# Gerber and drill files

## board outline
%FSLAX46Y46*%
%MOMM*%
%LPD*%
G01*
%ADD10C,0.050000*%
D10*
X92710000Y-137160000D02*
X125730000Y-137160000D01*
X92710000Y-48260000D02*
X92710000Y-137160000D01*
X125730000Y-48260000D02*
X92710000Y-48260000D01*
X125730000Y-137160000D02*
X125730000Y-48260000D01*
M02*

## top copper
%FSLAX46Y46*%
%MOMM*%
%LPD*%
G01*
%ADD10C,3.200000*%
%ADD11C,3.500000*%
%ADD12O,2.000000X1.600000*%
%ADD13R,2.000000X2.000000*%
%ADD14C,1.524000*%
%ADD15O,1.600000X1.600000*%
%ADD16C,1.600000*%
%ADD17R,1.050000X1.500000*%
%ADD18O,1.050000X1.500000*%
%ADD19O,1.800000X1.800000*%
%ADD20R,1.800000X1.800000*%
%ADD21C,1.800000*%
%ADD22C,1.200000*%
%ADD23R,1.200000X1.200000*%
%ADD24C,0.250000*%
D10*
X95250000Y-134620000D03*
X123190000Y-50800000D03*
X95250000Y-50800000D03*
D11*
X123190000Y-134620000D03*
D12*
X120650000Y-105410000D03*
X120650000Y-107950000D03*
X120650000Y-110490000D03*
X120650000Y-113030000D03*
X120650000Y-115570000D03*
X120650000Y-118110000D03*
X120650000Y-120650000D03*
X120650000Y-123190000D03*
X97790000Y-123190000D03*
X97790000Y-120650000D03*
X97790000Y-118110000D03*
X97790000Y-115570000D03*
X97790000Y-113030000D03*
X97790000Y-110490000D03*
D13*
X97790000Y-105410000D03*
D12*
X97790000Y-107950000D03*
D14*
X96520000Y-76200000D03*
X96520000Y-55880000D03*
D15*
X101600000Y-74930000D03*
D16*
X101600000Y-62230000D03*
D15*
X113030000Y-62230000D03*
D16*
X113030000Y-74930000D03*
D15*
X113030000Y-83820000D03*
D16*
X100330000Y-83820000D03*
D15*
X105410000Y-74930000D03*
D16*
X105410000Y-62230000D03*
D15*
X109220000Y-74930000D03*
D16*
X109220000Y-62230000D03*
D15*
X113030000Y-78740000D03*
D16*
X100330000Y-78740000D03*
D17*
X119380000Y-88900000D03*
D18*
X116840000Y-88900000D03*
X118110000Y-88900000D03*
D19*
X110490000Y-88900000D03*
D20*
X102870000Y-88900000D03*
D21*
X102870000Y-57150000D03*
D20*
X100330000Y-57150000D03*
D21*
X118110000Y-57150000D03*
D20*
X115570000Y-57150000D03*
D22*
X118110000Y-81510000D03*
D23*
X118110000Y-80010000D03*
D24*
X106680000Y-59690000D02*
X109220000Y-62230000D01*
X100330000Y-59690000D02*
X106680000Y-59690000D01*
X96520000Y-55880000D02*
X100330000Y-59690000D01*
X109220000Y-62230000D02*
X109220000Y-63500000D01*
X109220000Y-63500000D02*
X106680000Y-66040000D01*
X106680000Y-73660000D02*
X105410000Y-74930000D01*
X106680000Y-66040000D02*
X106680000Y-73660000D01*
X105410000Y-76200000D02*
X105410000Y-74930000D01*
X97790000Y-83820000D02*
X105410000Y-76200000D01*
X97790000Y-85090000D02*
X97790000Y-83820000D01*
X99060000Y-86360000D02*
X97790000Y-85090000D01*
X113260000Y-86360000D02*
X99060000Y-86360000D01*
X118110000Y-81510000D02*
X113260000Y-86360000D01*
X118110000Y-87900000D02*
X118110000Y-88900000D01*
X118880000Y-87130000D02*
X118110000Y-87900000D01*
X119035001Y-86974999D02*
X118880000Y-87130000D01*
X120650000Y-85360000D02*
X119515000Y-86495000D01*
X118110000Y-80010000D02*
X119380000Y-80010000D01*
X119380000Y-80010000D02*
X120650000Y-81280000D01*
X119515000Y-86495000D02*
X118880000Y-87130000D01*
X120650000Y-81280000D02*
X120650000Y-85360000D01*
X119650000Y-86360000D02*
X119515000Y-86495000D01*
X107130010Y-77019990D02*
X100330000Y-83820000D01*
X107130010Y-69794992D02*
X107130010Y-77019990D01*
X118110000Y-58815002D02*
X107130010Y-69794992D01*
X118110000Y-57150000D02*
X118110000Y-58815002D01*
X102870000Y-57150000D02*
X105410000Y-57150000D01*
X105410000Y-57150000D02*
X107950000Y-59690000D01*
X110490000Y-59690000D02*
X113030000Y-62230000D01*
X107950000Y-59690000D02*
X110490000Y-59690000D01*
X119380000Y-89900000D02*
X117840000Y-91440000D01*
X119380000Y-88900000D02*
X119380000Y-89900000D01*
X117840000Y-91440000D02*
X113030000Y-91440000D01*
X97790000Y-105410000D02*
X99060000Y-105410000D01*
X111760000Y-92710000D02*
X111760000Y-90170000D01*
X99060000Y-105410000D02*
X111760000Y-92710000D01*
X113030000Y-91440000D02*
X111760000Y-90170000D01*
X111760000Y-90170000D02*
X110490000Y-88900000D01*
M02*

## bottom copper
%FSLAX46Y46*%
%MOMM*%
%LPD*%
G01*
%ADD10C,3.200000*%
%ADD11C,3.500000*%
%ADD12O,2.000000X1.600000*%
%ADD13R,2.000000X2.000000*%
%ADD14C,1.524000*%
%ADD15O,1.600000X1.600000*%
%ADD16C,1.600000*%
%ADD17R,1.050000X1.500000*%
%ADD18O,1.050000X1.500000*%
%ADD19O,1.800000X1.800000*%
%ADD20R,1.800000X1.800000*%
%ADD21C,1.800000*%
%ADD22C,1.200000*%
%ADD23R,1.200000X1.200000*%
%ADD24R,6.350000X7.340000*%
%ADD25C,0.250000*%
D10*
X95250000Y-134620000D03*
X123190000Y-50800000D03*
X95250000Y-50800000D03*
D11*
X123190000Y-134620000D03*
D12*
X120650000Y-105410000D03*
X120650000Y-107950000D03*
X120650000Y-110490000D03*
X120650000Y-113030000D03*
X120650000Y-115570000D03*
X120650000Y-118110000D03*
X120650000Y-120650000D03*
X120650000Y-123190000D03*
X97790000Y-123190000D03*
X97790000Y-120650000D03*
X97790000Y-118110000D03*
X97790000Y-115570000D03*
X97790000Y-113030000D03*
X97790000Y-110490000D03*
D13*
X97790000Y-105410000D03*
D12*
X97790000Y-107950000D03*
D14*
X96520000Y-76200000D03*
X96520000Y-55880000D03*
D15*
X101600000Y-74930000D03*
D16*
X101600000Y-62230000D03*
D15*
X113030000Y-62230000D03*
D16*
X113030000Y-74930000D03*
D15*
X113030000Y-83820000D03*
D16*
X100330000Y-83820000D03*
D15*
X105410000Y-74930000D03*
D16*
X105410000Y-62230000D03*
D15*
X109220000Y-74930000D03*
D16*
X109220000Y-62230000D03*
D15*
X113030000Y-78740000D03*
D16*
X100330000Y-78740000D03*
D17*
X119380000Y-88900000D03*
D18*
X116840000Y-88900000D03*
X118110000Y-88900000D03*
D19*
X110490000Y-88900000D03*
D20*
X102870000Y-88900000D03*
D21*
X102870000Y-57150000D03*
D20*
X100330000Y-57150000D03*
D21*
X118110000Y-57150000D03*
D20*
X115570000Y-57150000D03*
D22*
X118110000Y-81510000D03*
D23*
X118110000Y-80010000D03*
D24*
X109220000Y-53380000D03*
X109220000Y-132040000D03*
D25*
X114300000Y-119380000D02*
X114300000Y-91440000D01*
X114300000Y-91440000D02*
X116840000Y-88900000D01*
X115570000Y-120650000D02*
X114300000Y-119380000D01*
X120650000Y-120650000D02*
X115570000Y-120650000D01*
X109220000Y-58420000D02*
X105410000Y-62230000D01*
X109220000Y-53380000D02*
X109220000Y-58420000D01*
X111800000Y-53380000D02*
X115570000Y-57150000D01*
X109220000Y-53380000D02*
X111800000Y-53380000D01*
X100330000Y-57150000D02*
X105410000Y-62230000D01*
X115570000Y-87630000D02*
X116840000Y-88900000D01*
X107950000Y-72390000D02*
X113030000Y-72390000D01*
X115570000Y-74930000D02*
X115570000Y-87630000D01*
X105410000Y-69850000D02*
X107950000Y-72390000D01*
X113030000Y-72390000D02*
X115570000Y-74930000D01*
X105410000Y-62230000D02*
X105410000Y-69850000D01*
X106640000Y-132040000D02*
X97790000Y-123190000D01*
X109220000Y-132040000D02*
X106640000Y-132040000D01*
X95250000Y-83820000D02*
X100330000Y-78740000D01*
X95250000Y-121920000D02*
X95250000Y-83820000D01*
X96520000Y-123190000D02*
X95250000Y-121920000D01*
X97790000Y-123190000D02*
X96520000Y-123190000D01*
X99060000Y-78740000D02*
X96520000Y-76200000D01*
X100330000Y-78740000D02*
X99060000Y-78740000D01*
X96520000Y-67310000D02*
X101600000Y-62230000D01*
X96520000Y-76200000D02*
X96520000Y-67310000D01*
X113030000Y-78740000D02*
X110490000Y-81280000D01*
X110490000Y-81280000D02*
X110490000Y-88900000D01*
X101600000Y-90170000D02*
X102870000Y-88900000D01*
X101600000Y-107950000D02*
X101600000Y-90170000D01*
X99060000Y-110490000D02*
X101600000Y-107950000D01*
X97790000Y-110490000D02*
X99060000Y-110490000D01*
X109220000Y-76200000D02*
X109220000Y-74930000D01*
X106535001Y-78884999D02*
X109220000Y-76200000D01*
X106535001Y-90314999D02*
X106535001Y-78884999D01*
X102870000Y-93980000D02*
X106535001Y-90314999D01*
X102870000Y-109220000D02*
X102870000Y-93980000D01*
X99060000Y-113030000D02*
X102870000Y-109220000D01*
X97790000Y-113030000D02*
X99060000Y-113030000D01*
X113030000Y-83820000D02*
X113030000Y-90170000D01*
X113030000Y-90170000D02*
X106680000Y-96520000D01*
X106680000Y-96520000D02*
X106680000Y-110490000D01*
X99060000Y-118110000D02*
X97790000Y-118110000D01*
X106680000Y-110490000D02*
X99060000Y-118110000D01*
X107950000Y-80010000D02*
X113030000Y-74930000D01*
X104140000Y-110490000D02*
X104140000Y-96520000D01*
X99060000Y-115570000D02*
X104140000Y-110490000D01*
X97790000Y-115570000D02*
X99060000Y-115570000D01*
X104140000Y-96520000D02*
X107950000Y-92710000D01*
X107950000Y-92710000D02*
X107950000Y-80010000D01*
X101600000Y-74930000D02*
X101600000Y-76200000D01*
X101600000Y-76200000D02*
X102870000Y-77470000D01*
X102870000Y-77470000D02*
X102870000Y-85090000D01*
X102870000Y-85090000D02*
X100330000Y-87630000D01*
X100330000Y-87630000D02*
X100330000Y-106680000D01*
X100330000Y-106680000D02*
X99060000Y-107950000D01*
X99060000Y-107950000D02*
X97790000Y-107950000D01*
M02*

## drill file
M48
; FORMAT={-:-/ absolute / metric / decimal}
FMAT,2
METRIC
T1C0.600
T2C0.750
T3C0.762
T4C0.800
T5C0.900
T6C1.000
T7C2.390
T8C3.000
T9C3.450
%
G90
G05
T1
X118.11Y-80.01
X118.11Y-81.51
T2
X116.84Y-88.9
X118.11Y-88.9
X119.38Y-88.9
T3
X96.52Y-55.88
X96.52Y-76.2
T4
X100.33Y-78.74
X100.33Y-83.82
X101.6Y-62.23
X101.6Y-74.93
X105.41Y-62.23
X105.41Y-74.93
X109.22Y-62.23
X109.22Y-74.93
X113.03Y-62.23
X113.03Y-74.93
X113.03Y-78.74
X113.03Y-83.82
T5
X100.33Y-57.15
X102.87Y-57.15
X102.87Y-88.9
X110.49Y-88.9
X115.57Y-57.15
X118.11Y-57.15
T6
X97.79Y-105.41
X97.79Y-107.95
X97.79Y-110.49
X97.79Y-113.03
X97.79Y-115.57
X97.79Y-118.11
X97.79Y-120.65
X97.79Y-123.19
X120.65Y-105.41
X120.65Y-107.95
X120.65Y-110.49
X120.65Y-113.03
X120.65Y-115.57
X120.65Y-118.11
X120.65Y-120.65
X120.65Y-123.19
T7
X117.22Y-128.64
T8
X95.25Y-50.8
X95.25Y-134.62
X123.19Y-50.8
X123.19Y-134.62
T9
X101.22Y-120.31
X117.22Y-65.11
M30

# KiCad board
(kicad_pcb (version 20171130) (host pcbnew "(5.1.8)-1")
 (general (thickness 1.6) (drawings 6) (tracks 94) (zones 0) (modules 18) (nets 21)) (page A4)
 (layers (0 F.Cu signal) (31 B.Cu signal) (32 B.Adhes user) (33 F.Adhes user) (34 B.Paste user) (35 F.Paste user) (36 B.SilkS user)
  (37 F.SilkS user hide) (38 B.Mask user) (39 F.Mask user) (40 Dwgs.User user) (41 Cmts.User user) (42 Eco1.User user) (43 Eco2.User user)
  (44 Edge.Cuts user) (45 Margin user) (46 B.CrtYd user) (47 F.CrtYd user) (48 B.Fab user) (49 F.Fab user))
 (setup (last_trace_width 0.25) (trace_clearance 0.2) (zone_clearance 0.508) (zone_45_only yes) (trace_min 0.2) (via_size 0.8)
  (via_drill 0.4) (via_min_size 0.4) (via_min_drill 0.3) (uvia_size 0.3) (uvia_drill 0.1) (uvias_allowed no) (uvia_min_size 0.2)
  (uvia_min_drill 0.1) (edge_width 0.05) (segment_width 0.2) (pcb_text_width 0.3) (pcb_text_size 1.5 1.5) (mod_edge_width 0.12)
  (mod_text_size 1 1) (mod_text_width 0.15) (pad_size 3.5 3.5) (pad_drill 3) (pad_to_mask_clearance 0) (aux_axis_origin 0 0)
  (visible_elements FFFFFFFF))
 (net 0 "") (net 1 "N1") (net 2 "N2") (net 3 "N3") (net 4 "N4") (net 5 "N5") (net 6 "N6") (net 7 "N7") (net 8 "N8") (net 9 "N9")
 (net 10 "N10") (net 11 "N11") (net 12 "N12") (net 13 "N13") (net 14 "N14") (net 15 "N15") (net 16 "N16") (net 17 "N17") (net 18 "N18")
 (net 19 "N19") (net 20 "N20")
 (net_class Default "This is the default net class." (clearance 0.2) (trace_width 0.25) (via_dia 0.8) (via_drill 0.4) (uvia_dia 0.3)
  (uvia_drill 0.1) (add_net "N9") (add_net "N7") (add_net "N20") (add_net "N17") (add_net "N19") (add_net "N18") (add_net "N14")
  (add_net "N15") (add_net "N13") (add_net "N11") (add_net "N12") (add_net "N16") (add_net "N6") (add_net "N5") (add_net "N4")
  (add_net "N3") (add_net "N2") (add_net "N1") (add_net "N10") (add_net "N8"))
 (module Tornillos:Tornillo (layer F.Cu) (at 95.25 132.08)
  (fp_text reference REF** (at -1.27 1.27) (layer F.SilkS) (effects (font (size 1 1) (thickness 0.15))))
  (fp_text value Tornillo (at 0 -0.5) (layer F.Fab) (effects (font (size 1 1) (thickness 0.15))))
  (pad "" np_thru_hole circle (at 0 2.54) (size 3.2 3.2) (drill 3) (layers *.Cu *.Mask)))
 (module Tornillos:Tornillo (layer F.Cu) (at 123.19 48.26)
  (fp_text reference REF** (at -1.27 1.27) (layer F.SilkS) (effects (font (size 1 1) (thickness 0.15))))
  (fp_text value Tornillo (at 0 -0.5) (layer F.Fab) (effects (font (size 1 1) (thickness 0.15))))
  (pad "" np_thru_hole circle (at 0 2.54) (size 3.2 3.2) (drill 3) (layers *.Cu *.Mask)))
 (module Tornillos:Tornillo (layer F.Cu) (at 95.25 48.26)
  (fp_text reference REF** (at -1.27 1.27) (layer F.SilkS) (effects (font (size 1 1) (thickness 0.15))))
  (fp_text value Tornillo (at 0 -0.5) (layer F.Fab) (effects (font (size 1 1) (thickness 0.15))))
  (pad "" np_thru_hole circle (at 0 2.54) (size 3.2 3.2) (drill 3) (layers *.Cu *.Mask)))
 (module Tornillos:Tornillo (layer F.Cu) (at 123.19 132.08)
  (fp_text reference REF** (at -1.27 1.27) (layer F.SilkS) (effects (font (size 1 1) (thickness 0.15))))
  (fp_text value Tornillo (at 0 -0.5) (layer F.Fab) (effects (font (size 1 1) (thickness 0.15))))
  (pad "" np_thru_hole circle (at 0 2.54) (size 3.5 3.5) (drill 3) (layers *.Cu *.Mask)))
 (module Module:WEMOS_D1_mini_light (layer F.Cu) (at 97.79 105.41)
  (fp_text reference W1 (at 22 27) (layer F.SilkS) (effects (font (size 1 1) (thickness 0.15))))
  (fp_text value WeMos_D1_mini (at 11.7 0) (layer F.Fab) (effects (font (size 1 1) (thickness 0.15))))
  (pad 16 thru_hole oval (at 22.86 0) (size 2 1.6) (drill 1) (layers *.Cu *.Mask) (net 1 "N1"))
  (pad 15 thru_hole oval (at 22.86 2.54) (size 2 1.6) (drill 1) (layers *.Cu *.Mask) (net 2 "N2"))
  (pad 14 thru_hole oval (at 22.86 5.08) (size 2 1.6) (drill 1) (layers *.Cu *.Mask) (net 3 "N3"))
  (pad 13 thru_hole oval (at 22.86 7.62) (size 2 1.6) (drill 1) (layers *.Cu *.Mask) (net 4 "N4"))
  (pad 12 thru_hole oval (at 22.86 10.16) (size 2 1.6) (drill 1) (layers *.Cu *.Mask) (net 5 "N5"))
  (pad 11 thru_hole oval (at 22.86 12.7) (size 2 1.6) (drill 1) (layers *.Cu *.Mask) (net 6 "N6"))
  (pad 10 thru_hole oval (at 22.86 15.24) (size 2 1.6) (drill 1) (layers *.Cu *.Mask) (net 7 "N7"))
  (pad 9 thru_hole oval (at 22.86 17.78) (size 2 1.6) (drill 1) (layers *.Cu *.Mask) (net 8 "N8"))
  (pad 8 thru_hole oval (at 0 17.78) (size 2 1.6) (drill 1) (layers *.Cu *.Mask) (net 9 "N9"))
  (pad 7 thru_hole oval (at 0 15.24) (size 2 1.6) (drill 1) (layers *.Cu *.Mask) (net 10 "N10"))
  (pad 6 thru_hole oval (at 0 12.7) (size 2 1.6) (drill 1) (layers *.Cu *.Mask) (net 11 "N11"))
  (pad 5 thru_hole oval (at 0 10.16) (size 2 1.6) (drill 1) (layers *.Cu *.Mask) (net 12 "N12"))
  (pad 4 thru_hole oval (at 0 7.62) (size 2 1.6) (drill 1) (layers *.Cu *.Mask) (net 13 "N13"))
  (pad 3 thru_hole oval (at 0 5.08) (size 2 1.6) (drill 1) (layers *.Cu *.Mask) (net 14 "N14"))
  (pad 1 thru_hole rect (at 0 0) (size 2 2) (drill 1) (layers *.Cu *.Mask) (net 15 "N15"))
  (pad 2 thru_hole oval (at 0 2.54) (size 2 1.6) (drill 1) (layers *.Cu *.Mask) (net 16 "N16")))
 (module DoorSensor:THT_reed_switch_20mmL (layer F.Cu) (at 100.33 63.5 270)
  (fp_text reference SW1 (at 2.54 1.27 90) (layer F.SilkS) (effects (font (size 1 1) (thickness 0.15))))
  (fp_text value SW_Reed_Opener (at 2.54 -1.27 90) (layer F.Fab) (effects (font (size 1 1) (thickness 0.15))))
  (pad 2 thru_hole circle (at 12.7 3.81 270) (size 1.524 1.524) (drill 0.762) (layers *.Cu *.Mask) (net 9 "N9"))
  (pad 1 thru_hole circle (at -7.62 3.81 270) (size 1.524 1.524) (drill 0.762) (layers *.Cu *.Mask) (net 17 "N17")))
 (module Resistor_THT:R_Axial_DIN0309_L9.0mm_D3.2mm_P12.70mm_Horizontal (layer F.Cu) (at 101.6 62.23 270)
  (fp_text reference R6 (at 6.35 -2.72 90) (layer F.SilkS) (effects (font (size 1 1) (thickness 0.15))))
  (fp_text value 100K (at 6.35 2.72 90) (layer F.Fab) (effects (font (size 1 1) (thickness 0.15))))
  (pad 2 thru_hole oval (at 12.7 0 270) (size 1.6 1.6) (drill 0.8) (layers *.Cu *.Mask) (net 16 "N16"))
  (pad 1 thru_hole circle (at 0 0 270) (size 1.6 1.6) (drill 0.8) (layers *.Cu *.Mask) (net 9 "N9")))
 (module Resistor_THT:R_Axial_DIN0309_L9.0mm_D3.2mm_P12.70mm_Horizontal (layer F.Cu) (at 113.03 74.93 90)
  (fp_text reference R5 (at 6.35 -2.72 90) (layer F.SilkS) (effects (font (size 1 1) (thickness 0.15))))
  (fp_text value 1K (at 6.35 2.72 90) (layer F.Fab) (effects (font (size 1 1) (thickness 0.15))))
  (pad 2 thru_hole oval (at 12.7 0 90) (size 1.6 1.6) (drill 0.8) (layers *.Cu *.Mask) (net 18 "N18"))
  (pad 1 thru_hole circle (at 0 0 90) (size 1.6 1.6) (drill 0.8) (layers *.Cu *.Mask) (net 12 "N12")))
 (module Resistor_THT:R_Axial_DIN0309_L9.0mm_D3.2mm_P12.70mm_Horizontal (layer F.Cu) (at 100.33 83.82)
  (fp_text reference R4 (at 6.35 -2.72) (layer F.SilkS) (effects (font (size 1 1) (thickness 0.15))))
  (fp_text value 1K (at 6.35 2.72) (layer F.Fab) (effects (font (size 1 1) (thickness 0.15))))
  (pad 2 thru_hole oval (at 12.7 0) (size 1.6 1.6) (drill 0.8) (layers *.Cu *.Mask) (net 11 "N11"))
  (pad 1 thru_hole circle (at 0 0) (size 1.6 1.6) (drill 0.8) (layers *.Cu *.Mask) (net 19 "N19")))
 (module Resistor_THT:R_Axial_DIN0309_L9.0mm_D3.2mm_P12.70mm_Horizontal (layer F.Cu) (at 105.41 62.23 270)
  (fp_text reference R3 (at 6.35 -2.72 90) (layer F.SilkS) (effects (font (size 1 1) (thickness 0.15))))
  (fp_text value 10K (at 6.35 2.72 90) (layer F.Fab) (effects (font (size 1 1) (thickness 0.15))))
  (pad 2 thru_hole oval (at 12.7 0 270) (size 1.6 1.6) (drill 0.8) (layers *.Cu *.Mask) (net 17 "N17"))
  (pad 1 thru_hole circle (at 0 0 270) (size 1.6 1.6) (drill 0.8) (layers *.Cu *.Mask) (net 7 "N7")))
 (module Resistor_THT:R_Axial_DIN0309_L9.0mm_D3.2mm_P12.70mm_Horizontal (layer F.Cu) (at 109.22 62.23 270)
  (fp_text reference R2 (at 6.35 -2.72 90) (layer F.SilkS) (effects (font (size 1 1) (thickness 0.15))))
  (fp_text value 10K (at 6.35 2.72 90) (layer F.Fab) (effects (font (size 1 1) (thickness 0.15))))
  (pad 2 thru_hole oval (at 12.7 0 270) (size 1.6 1.6) (drill 0.8) (layers *.Cu *.Mask) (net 13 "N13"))
  (pad 1 thru_hole circle (at 0 0 270) (size 1.6 1.6) (drill 0.8) (layers *.Cu *.Mask) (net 17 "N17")))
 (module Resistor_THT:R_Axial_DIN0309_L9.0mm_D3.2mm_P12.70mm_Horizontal (layer F.Cu) (at 100.33 78.74)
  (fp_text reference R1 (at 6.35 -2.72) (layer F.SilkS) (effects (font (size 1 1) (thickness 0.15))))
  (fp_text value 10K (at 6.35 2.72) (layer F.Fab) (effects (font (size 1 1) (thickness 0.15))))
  (pad 2 thru_hole oval (at 12.7 0) (size 1.6 1.6) (drill 0.8) (layers *.Cu *.Mask) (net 15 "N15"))
  (pad 1 thru_hole circle (at 0 0) (size 1.6 1.6) (drill 0.8) (layers *.Cu *.Mask) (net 9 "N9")))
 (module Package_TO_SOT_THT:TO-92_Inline (layer F.Cu) (at 119.38 88.9 180)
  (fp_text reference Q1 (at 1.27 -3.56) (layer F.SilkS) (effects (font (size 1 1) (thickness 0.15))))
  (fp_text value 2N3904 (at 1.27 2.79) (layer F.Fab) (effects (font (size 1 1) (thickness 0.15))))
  (pad 1 thru_hole rect (at 0 0 180) (size 1.05 1.5) (drill 0.75) (layers *.Cu *.Mask) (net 15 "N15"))
  (pad 3 thru_hole oval (at 2.54 0 180) (size 1.05 1.5) (drill 0.75) (layers *.Cu *.Mask) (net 7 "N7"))
  (pad 2 thru_hole oval (at 1.27 0 180) (size 1.05 1.5) (drill 0.75) (layers *.Cu *.Mask) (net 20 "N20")))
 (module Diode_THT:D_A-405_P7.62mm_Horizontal (layer F.Cu) (at 102.87 88.9)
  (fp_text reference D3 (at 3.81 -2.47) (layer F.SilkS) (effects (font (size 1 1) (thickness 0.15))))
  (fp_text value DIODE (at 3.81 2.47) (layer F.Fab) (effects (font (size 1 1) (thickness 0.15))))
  (pad 2 thru_hole oval (at 7.62 0) (size 1.8 1.8) (drill 0.9) (layers *.Cu *.Mask) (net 15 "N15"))
  (pad 1 thru_hole rect (at 0 0) (size 1.8 1.8) (drill 0.9) (layers *.Cu *.Mask) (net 14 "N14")))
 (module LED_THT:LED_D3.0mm (layer F.Cu) (at 100.33 57.15)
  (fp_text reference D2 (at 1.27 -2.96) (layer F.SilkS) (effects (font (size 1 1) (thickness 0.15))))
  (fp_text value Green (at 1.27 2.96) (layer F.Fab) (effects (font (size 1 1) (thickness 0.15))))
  (pad 2 thru_hole circle (at 2.54 0) (size 1.8 1.8) (drill 0.9) (layers *.Cu *.Mask) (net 18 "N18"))
  (pad 1 thru_hole rect (at 0 0) (size 1.8 1.8) (drill 0.9) (layers *.Cu *.Mask) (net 7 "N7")))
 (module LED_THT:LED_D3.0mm (layer F.Cu) (at 115.57 57.15)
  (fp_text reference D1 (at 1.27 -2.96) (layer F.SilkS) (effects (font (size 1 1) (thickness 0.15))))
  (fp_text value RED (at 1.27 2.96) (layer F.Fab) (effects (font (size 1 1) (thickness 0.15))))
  (pad 2 thru_hole circle (at 2.54 0) (size 1.8 1.8) (drill 0.9) (layers *.Cu *.Mask) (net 19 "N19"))
  (pad 1 thru_hole rect (at 0 0) (size 1.8 1.8) (drill 0.9) (layers *.Cu *.Mask) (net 7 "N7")))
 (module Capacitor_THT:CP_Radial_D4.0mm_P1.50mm (layer F.Cu) (at 118.11 80.01 270)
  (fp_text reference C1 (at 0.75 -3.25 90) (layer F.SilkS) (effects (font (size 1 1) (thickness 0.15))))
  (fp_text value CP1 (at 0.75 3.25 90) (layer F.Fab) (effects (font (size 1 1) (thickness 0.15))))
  (pad 2 thru_hole circle (at 1.5 0 270) (size 1.2 1.2) (drill 0.6) (layers *.Cu *.Mask) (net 17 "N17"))
  (pad 1 thru_hole rect (at 0 0 270) (size 1.2 1.2) (drill 0.6) (layers *.Cu *.Mask) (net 20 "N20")))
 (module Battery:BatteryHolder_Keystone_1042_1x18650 (layer B.Cu) (at 109.22 92.71 90)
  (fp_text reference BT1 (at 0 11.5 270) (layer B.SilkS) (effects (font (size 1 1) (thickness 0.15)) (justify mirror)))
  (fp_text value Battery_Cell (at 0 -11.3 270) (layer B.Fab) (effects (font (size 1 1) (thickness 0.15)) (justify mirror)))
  (pad "" np_thru_hole circle (at -35.93 8 90) (size 2.39 2.39) (drill 2.39) (layers *.Cu *.Mask))
  (pad "" np_thru_hole circle (at -27.6 -8 90) (size 3.45 3.45) (drill 3.45) (layers *.Cu *.Mask))
  (pad "" np_thru_hole circle (at 27.6 8 90) (size 3.45 3.45) (drill 3.45) (layers *.Cu *.Mask))
  (pad 2 smd rect (at 39.33 0 90) (size 7.34 6.35) (layers B.Cu B.Paste B.Mask) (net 7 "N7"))
  (pad 1 smd rect (at -39.33 0 90) (size 7.34 6.35) (layers B.Cu B.Paste B.Mask) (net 9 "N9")))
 (gr_line (start 92.71 137.16) (end 125.73 137.16) (layer Edge.Cuts) (width 0.05))
 (gr_line (start 92.71 48.26) (end 92.71 137.16) (layer Edge.Cuts) (width 0.05))
 (gr_line (start 125.73 48.26) (end 92.71 48.26) (layer Edge.Cuts) (width 0.05))
 (gr_line (start 125.73 137.16) (end 125.73 48.26) (layer Edge.Cuts) (width 0.05))
 (segment (start 114.3 119.38) (end 114.3 91.44) (width 0.25) (layer B.Cu) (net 7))
 (segment (start 114.3 91.44) (end 116.84 88.9) (width 0.25) (layer B.Cu) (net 7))
 (segment (start 115.57 120.65) (end 114.3 119.38) (width 0.25) (layer B.Cu) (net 7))
 (segment (start 120.65 120.65) (end 115.57 120.65) (width 0.25) (layer B.Cu) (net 7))
 (segment (start 109.22 58.42) (end 105.41 62.23) (width 0.25) (layer B.Cu) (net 7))
 (segment (start 109.22 53.38) (end 109.22 58.42) (width 0.25) (layer B.Cu) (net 7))
 (segment (start 111.8 53.38) (end 115.57 57.15) (width 0.25) (layer B.Cu) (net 7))
 (segment (start 109.22 53.38) (end 111.8 53.38) (width 0.25) (layer B.Cu) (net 7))
 (segment (start 100.33 57.15) (end 105.41 62.23) (width 0.25) (layer B.Cu) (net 7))
 (segment (start 115.57 87.63) (end 116.84 88.9) (width 0.25) (layer B.Cu) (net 7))
 (segment (start 107.95 72.39) (end 113.03 72.39) (width 0.25) (layer B.Cu) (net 7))
 (segment (start 115.57 74.93) (end 115.57 87.63) (width 0.25) (layer B.Cu) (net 7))
 (segment (start 105.41 69.85) (end 107.95 72.39) (width 0.25) (layer B.Cu) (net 7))
 (segment (start 113.03 72.39) (end 115.57 74.93) (width 0.25) (layer B.Cu) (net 7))
 (segment (start 105.41 62.23) (end 105.41 69.85) (width 0.25) (layer B.Cu) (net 7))
 (segment (start 106.64 132.04) (end 97.79 123.19) (width 0.25) (layer B.Cu) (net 9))
 (segment (start 109.22 132.04) (end 106.64 132.04) (width 0.25) (layer B.Cu) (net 9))
 (segment (start 95.25 83.82) (end 100.33 78.74) (width 0.25) (layer B.Cu) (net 9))
 (segment (start 95.25 121.92) (end 95.25 83.82) (width 0.25) (layer B.Cu) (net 9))
 (segment (start 96.52 123.19) (end 95.25 121.92) (width 0.25) (layer B.Cu) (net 9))
 (segment (start 97.79 123.19) (end 96.52 123.19) (width 0.25) (layer B.Cu) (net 9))
 (segment (start 99.06 78.74) (end 96.52 76.2) (width 0.25) (layer B.Cu) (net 9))
 (segment (start 100.33 78.74) (end 99.06 78.74) (width 0.25) (layer B.Cu) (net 9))
 (segment (start 96.52 67.31) (end 101.6 62.23) (width 0.25) (layer B.Cu) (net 9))
 (segment (start 96.52 76.2) (end 96.52 67.31) (width 0.25) (layer B.Cu) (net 9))
 (segment (start 106.68 59.69) (end 109.22 62.23) (width 0.25) (layer F.Cu) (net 17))
 (segment (start 100.33 59.69) (end 106.68 59.69) (width 0.25) (layer F.Cu) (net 17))
 (segment (start 96.52 55.88) (end 100.33 59.69) (width 0.25) (layer F.Cu) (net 17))
 (segment (start 109.22 62.23) (end 109.22 63.5) (width 0.25) (layer F.Cu) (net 17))
 (segment (start 109.22 63.5) (end 106.68 66.04) (width 0.25) (layer F.Cu) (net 17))
 (segment (start 106.68 73.66) (end 105.41 74.93) (width 0.25) (layer F.Cu) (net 17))
 (segment (start 106.68 66.04) (end 106.68 73.66) (width 0.25) (layer F.Cu) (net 17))
 (segment (start 105.41 76.2) (end 105.41 74.93) (width 0.25) (layer F.Cu) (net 17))
 (segment (start 97.79 83.82) (end 105.41 76.2) (width 0.25) (layer F.Cu) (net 17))
 (segment (start 97.79 85.09) (end 97.79 83.82) (width 0.25) (layer F.Cu) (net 17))
 (segment (start 99.06 86.36) (end 97.79 85.09) (width 0.25) (layer F.Cu) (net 17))
 (segment (start 113.26 86.36) (end 99.06 86.36) (width 0.25) (layer F.Cu) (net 17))
 (segment (start 118.11 81.51) (end 113.26 86.36) (width 0.25) (layer F.Cu) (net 17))
 (segment (start 118.11 87.9) (end 118.11 88.9) (width 0.25) (layer F.Cu) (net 20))
 (segment (start 118.88 87.13) (end 118.11 87.9) (width 0.25) (layer F.Cu) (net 20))
 (segment (start 119.035001 86.974999) (end 118.88 87.13) (width 0.25) (layer F.Cu) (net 20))
 (segment (start 120.65 85.36) (end 119.515 86.495) (width 0.25) (layer F.Cu) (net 20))
 (segment (start 118.11 80.01) (end 119.38 80.01) (width 0.25) (layer F.Cu) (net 20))
 (segment (start 119.38 80.01) (end 120.65 81.28) (width 0.25) (layer F.Cu) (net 20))
 (segment (start 119.515 86.495) (end 118.88 87.13) (width 0.25) (layer F.Cu) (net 20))
 (segment (start 120.65 81.28) (end 120.65 85.36) (width 0.25) (layer F.Cu) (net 20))
 (segment (start 119.65 86.36) (end 119.515 86.495) (width 0.25) (layer F.Cu) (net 20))
 (segment (start 107.13001 77.01999) (end 100.33 83.82) (width 0.25) (layer F.Cu) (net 19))
 (segment (start 107.13001 69.794992) (end 107.13001 77.01999) (width 0.25) (layer F.Cu) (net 19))
 (segment (start 118.11 58.815002) (end 107.13001 69.794992) (width 0.25) (layer F.Cu) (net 19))
 (segment (start 118.11 57.15) (end 118.11 58.815002) (width 0.25) (layer F.Cu) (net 19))
 (segment (start 102.87 57.15) (end 105.41 57.15) (width 0.25) (layer F.Cu) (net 18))
 (segment (start 105.41 57.15) (end 107.95 59.69) (width 0.25) (layer F.Cu) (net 18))
 (segment (start 110.49 59.69) (end 113.03 62.23) (width 0.25) (layer F.Cu) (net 18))
 (segment (start 107.95 59.69) (end 110.49 59.69) (width 0.25) (layer F.Cu) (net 18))
 (segment (start 119.38 89.9) (end 117.84 91.44) (width 0.25) (layer F.Cu) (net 15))
 (segment (start 119.38 88.9) (end 119.38 89.9) (width 0.25) (layer F.Cu) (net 15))
 (segment (start 117.84 91.44) (end 113.03 91.44) (width 0.25) (layer F.Cu) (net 15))
 (segment (start 113.03 78.74) (end 110.49 81.28) (width 0.25) (layer B.Cu) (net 15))
 (segment (start 110.49 81.28) (end 110.49 88.9) (width 0.25) (layer B.Cu) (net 15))
 (segment (start 97.79 105.41) (end 99.06 105.41) (width 0.25) (layer F.Cu) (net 15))
 (segment (start 111.76 92.71) (end 111.76 90.17) (width 0.25) (layer F.Cu) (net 15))
 (segment (start 99.06 105.41) (end 111.76 92.71) (width 0.25) (layer F.Cu) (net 15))
 (segment (start 113.03 91.44) (end 111.76 90.17) (width 0.25) (layer F.Cu) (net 15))
 (segment (start 111.76 90.17) (end 110.49 88.9) (width 0.25) (layer F.Cu) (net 15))
 (segment (start 101.6 90.17) (end 102.87 88.9) (width 0.25) (layer B.Cu) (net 14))
 (segment (start 101.6 107.95) (end 101.6 90.17) (width 0.25) (layer B.Cu) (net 14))
 (segment (start 99.06 110.49) (end 101.6 107.95) (width 0.25) (layer B.Cu) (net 14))
 (segment (start 97.79 110.49) (end 99.06 110.49) (width 0.25) (layer B.Cu) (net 14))
 (segment (start 109.22 76.2) (end 109.22 74.93) (width 0.25) (layer B.Cu) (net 13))
 (segment (start 106.535001 78.884999) (end 109.22 76.2) (width 0.25) (layer B.Cu) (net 13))
 (segment (start 106.535001 90.314999) (end 106.535001 78.884999) (width 0.25) (layer B.Cu) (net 13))
 (segment (start 102.87 93.98) (end 106.535001 90.314999) (width 0.25) (layer B.Cu) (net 13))
 (segment (start 102.87 109.22) (end 102.87 93.98) (width 0.25) (layer B.Cu) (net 13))
 (segment (start 99.06 113.03) (end 102.87 109.22) (width 0.25) (layer B.Cu) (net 13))
 (segment (start 97.79 113.03) (end 99.06 113.03) (width 0.25) (layer B.Cu) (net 13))
 (segment (start 113.03 83.82) (end 113.03 90.17) (width 0.25) (layer B.Cu) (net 11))
 (segment (start 113.03 90.17) (end 106.68 96.52) (width 0.25) (layer B.Cu) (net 11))
 (segment (start 106.68 96.52) (end 106.68 110.49) (width 0.25) (layer B.Cu) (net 11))
 (segment (start 99.06 118.11) (end 97.79 118.11) (width 0.25) (layer B.Cu) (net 11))
 (segment (start 106.68 110.49) (end 99.06 118.11) (width 0.25) (layer B.Cu) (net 11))
 (segment (start 107.95 80.01) (end 113.03 74.93) (width 0.25) (layer B.Cu) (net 12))
 (segment (start 104.14 110.49) (end 104.14 96.52) (width 0.25) (layer B.Cu) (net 12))
 (segment (start 99.06 115.57) (end 104.14 110.49) (width 0.25) (layer B.Cu) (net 12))
 (segment (start 97.79 115.57) (end 99.06 115.57) (width 0.25) (layer B.Cu) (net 12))
 (segment (start 104.14 96.52) (end 107.95 92.71) (width 0.25) (layer B.Cu) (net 12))
 (segment (start 107.95 92.71) (end 107.95 80.01) (width 0.25) (layer B.Cu) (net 12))
 (segment (start 101.6 74.93) (end 101.6 76.2) (width 0.25) (layer B.Cu) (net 16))
 (segment (start 101.6 76.2) (end 102.87 77.47) (width 0.25) (layer B.Cu) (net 16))
 (segment (start 102.87 77.47) (end 102.87 85.09) (width 0.25) (layer B.Cu) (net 16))
 (segment (start 102.87 85.09) (end 100.33 87.63) (width 0.25) (layer B.Cu) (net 16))
 (segment (start 100.33 87.63) (end 100.33 106.68) (width 0.25) (layer B.Cu) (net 16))
 (segment (start 100.33 106.68) (end 99.06 107.95) (width 0.25) (layer B.Cu) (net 16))
 (segment (start 99.06 107.95) (end 97.79 107.95) (width 0.25) (layer B.Cu) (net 16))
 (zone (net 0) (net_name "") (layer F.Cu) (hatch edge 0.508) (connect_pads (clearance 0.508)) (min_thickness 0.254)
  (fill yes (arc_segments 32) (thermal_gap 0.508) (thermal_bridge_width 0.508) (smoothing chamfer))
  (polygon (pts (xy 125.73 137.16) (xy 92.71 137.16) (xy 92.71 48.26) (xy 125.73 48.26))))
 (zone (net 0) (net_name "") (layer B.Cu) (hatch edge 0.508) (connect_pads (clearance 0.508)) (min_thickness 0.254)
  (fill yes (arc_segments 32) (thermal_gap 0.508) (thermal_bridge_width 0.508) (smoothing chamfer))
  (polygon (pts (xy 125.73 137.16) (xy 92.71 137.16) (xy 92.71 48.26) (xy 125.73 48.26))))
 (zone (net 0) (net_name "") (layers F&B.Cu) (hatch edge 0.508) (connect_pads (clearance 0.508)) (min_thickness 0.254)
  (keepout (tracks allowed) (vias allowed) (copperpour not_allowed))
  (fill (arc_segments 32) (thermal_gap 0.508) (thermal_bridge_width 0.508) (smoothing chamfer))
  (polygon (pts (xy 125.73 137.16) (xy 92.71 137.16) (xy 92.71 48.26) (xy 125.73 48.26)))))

